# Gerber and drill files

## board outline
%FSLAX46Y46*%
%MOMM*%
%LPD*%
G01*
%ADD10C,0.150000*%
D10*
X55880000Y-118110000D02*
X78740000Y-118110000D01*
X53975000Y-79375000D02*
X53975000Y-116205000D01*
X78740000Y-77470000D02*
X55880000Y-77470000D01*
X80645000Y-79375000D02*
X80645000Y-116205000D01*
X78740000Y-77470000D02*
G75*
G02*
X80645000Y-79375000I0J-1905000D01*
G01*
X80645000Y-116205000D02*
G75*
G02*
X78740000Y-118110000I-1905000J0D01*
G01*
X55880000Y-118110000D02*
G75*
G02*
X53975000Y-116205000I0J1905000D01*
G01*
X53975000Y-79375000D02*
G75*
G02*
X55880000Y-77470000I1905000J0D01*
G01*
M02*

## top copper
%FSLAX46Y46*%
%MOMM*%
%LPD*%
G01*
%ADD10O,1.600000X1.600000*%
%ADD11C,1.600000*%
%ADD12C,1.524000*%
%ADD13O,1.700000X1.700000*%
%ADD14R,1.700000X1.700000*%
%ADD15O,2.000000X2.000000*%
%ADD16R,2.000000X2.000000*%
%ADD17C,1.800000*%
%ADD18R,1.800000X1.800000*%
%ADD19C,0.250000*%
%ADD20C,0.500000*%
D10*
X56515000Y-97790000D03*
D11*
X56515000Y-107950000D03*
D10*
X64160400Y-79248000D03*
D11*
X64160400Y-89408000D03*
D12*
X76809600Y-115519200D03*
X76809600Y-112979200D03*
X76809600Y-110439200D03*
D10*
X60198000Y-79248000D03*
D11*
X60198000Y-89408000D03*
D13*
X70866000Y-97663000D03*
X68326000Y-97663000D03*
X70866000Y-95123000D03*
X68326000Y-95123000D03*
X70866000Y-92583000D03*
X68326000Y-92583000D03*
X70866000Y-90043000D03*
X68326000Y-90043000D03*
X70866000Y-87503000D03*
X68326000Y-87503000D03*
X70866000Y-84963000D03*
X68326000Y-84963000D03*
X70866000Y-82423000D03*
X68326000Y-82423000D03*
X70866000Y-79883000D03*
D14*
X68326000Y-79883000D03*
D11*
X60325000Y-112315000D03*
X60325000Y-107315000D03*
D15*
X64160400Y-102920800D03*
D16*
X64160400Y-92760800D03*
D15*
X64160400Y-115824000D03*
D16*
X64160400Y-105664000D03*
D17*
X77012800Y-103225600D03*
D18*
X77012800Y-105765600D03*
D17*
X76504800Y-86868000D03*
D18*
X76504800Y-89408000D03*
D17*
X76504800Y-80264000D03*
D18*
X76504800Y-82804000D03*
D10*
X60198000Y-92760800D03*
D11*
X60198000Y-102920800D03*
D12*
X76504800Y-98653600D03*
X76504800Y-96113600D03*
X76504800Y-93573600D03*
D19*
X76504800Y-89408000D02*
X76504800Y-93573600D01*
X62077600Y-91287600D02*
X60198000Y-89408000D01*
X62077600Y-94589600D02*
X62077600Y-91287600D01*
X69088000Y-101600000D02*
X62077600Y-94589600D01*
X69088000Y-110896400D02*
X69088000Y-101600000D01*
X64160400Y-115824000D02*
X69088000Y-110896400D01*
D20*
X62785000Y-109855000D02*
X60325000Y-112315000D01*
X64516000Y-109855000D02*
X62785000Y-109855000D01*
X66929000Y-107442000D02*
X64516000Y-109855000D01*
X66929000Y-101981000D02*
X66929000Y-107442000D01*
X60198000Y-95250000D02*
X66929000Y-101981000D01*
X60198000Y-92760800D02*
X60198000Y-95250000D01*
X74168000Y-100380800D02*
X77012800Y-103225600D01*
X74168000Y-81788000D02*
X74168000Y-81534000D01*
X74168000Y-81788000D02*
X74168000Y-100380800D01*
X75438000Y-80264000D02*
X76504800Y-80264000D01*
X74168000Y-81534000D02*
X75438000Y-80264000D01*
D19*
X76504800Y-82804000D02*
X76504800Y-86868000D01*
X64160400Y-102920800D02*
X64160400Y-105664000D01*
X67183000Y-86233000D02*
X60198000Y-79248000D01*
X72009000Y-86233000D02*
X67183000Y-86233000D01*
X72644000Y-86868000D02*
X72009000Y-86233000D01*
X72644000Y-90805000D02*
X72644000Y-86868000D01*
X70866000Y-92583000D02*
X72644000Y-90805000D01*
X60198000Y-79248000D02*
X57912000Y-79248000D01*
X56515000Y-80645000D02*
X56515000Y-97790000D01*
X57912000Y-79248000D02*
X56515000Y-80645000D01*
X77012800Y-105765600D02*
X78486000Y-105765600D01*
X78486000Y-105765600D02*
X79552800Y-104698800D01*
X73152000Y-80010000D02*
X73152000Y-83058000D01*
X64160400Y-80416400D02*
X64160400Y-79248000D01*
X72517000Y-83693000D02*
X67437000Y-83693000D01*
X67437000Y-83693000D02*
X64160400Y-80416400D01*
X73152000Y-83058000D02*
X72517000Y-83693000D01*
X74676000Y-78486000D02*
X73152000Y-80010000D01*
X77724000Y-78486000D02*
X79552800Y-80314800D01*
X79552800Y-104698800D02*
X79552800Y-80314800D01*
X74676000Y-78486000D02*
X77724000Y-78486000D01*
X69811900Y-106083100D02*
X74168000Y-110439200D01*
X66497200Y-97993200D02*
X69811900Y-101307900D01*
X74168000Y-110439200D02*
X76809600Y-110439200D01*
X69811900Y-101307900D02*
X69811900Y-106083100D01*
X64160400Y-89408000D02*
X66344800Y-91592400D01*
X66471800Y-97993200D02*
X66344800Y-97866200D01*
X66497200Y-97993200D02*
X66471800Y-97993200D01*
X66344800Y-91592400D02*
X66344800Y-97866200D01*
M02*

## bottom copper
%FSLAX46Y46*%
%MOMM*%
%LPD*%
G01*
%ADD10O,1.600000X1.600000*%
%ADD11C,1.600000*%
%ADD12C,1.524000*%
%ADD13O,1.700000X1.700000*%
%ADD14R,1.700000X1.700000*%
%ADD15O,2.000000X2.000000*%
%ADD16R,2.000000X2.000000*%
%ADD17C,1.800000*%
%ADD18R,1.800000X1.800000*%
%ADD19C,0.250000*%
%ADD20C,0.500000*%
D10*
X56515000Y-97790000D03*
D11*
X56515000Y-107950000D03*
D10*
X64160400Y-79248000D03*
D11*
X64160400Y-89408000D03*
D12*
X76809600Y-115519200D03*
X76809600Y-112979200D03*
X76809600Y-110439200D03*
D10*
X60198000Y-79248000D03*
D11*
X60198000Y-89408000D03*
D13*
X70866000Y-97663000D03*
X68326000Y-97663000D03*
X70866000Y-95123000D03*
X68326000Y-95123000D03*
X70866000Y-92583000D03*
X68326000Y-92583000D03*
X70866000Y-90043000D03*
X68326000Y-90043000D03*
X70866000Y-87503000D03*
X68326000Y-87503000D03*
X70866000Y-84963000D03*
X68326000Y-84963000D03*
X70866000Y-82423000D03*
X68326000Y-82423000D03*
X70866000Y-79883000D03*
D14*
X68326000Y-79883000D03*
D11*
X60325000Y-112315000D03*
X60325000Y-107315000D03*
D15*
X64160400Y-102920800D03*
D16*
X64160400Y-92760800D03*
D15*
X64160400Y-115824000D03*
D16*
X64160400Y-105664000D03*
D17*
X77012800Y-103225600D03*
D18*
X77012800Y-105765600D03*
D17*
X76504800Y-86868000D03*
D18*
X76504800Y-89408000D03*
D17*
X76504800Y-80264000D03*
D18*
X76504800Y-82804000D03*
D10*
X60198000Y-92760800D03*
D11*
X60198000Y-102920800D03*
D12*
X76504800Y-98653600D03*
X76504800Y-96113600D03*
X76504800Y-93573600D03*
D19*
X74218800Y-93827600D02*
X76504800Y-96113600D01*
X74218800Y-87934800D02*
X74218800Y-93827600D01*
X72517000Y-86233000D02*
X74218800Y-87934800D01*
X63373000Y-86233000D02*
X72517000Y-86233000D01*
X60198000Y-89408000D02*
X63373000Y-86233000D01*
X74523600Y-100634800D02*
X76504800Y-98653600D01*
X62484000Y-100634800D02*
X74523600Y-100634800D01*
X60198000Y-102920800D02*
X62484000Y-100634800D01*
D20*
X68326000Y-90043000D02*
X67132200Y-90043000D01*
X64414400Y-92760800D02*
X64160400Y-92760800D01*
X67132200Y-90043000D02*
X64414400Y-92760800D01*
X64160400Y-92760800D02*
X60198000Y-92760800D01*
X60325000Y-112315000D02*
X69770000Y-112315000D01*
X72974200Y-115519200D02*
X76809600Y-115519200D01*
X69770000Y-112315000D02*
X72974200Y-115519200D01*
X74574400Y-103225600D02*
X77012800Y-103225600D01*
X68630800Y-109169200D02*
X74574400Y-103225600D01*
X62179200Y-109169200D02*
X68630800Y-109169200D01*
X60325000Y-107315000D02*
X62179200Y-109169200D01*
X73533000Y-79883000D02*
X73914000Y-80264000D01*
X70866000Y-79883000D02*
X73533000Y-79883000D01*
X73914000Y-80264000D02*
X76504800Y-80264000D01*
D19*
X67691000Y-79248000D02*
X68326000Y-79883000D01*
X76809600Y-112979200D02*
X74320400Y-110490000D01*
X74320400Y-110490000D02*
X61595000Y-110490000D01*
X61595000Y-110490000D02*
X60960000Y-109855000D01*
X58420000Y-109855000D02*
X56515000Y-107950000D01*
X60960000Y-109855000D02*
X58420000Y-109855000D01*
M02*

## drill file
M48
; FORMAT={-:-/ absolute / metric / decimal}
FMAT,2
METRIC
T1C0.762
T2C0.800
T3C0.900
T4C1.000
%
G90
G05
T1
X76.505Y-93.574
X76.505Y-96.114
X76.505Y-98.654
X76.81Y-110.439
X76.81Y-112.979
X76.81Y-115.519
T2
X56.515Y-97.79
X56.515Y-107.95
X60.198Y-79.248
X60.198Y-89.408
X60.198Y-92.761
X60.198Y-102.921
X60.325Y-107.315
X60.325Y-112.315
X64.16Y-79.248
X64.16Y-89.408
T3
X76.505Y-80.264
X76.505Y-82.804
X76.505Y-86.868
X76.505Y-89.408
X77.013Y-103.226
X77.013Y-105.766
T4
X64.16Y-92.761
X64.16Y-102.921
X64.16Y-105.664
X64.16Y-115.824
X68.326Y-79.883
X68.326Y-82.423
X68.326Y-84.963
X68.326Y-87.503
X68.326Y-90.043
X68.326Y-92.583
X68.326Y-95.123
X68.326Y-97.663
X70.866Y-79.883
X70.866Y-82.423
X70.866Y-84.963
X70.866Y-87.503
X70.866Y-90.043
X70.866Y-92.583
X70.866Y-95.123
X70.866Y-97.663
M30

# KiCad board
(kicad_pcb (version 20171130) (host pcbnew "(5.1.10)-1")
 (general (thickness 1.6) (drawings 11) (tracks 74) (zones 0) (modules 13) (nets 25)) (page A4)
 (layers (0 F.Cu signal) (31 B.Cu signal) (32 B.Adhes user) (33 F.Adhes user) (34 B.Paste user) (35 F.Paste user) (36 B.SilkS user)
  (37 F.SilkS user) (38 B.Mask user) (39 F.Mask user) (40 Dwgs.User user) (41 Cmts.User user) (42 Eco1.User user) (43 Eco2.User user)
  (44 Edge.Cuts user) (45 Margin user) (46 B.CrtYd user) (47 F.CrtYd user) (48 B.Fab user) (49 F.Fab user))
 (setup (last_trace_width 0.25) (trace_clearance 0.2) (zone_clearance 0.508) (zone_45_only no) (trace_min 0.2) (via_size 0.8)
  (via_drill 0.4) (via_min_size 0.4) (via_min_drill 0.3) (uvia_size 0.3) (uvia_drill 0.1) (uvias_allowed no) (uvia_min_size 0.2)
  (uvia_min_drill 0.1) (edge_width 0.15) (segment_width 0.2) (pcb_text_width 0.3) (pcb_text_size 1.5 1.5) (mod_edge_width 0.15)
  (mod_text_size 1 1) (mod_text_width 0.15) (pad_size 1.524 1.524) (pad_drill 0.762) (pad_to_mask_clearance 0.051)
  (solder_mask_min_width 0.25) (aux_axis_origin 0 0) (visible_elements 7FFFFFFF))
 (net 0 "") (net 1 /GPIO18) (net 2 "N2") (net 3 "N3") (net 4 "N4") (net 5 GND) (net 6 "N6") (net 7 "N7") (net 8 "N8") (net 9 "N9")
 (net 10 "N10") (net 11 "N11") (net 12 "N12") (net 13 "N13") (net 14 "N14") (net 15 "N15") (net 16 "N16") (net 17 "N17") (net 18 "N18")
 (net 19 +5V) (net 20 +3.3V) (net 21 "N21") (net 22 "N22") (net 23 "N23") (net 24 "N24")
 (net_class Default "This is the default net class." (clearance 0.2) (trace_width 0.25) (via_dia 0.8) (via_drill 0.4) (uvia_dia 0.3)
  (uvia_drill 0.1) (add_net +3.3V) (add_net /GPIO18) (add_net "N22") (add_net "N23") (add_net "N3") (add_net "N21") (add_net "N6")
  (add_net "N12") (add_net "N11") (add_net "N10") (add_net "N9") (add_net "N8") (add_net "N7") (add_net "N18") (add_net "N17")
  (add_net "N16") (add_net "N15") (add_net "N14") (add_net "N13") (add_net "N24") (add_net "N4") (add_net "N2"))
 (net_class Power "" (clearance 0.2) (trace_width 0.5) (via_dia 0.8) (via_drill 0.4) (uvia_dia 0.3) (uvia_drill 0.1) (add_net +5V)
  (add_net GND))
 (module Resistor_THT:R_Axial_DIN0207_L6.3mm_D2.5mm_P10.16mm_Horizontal (layer F.Cu) (at 56.515 107.95 90)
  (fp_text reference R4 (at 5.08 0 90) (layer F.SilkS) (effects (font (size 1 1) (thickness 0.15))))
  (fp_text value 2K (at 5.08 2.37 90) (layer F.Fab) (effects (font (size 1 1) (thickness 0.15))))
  (pad 2 thru_hole oval (at 10.16 0 90) (size 1.6 1.6) (drill 0.8) (layers *.Cu *.Mask) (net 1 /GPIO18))
  (pad 1 thru_hole circle (at 0 0 90) (size 1.6 1.6) (drill 0.8) (layers *.Cu *.Mask) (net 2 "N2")))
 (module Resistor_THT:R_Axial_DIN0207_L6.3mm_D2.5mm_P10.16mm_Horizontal (layer F.Cu) (at 64.1604 89.408 90)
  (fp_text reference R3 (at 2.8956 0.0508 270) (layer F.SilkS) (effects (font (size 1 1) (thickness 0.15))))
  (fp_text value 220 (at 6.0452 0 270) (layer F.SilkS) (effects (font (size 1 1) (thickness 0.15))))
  (pad 2 thru_hole oval (at 10.16 0 90) (size 1.6 1.6) (drill 0.8) (layers *.Cu *.Mask) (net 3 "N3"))
  (pad 1 thru_hole circle (at 0 0 90) (size 1.6 1.6) (drill 0.8) (layers *.Cu *.Mask) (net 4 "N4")))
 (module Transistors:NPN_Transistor (layer F.Cu) (at 76.8096 110.4392 270)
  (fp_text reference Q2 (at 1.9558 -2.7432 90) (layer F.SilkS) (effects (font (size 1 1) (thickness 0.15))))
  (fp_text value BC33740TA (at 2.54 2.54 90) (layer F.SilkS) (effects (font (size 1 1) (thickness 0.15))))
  (pad 3 thru_hole circle (at 5.08 0 270) (size 1.524 1.524) (drill 0.762) (layers *.Cu *.Mask) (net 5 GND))
  (pad 2 thru_hole circle (at 2.54 0 270) (size 1.524 1.524) (drill 0.762) (layers *.Cu *.Mask) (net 2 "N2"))
  (pad 1 thru_hole circle (at 0 0 270) (size 1.524 1.524) (drill 0.762) (layers *.Cu *.Mask) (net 4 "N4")))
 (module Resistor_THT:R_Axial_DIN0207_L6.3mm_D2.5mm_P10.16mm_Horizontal (layer F.Cu) (at 60.198 89.408 90)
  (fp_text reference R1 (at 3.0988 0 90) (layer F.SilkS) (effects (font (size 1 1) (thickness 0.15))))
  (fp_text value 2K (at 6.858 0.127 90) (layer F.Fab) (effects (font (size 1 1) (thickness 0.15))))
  (pad 2 thru_hole oval (at 10.16 0 90) (size 1.6 1.6) (drill 0.8) (layers *.Cu *.Mask) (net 1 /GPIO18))
  (pad 1 thru_hole circle (at 0 0 90) (size 1.6 1.6) (drill 0.8) (layers *.Cu *.Mask) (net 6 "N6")))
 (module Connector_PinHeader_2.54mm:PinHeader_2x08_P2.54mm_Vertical (layer F.Cu) (at 68.326 79.883)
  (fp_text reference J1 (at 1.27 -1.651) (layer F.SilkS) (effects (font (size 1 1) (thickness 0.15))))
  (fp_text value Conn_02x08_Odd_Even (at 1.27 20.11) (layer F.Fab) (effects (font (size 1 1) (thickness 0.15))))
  (pad 16 thru_hole oval (at 2.54 17.78) (size 1.7 1.7) (drill 1) (layers *.Cu *.Mask) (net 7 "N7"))
  (pad 15 thru_hole oval (at 0 17.78) (size 1.7 1.7) (drill 1) (layers *.Cu *.Mask) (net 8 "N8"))
  (pad 14 thru_hole oval (at 2.54 15.24) (size 1.7 1.7) (drill 1) (layers *.Cu *.Mask) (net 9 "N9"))
  (pad 13 thru_hole oval (at 0 15.24) (size 1.7 1.7) (drill 1) (layers *.Cu *.Mask) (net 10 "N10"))
  (pad 12 thru_hole oval (at 2.54 12.7) (size 1.7 1.7) (drill 1) (layers *.Cu *.Mask) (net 1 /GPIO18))
  (pad 11 thru_hole oval (at 0 12.7) (size 1.7 1.7) (drill 1) (layers *.Cu *.Mask) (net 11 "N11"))
  (pad 10 thru_hole oval (at 2.54 10.16) (size 1.7 1.7) (drill 1) (layers *.Cu *.Mask) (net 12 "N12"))
  (pad 9 thru_hole oval (at 0 10.16) (size 1.7 1.7) (drill 1) (layers *.Cu *.Mask) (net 5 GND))
  (pad 8 thru_hole oval (at 2.54 7.62) (size 1.7 1.7) (drill 1) (layers *.Cu *.Mask) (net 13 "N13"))
  (pad 7 thru_hole oval (at 0 7.62) (size 1.7 1.7) (drill 1) (layers *.Cu *.Mask) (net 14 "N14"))
  (pad 6 thru_hole oval (at 2.54 5.08) (size 1.7 1.7) (drill 1) (layers *.Cu *.Mask) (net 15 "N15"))
  (pad 5 thru_hole oval (at 0 5.08) (size 1.7 1.7) (drill 1) (layers *.Cu *.Mask) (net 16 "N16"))
  (pad 4 thru_hole oval (at 2.54 2.54) (size 1.7 1.7) (drill 1) (layers *.Cu *.Mask) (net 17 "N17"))
  (pad 3 thru_hole oval (at 0 2.54) (size 1.7 1.7) (drill 1) (layers *.Cu *.Mask) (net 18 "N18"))
  (pad 2 thru_hole oval (at 2.54 0) (size 1.7 1.7) (drill 1) (layers *.Cu *.Mask) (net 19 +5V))
  (pad 1 thru_hole rect (at 0 0) (size 1.7 1.7) (drill 1) (layers *.Cu *.Mask) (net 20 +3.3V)))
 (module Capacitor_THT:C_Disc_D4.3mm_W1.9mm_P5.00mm (layer F.Cu) (at 60.325 107.315 270)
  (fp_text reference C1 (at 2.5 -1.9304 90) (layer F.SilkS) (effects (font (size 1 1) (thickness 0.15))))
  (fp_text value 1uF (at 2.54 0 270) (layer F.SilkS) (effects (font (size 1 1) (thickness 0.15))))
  (pad 2 thru_hole circle (at 5 0 270) (size 1.6 1.6) (drill 0.8) (layers *.Cu *.Mask) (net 5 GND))
  (pad 1 thru_hole circle (at 0 0 270) (size 1.6 1.6) (drill 0.8) (layers *.Cu *.Mask) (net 19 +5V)))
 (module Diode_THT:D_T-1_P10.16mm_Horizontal (layer F.Cu) (at 64.1604 92.7608 270)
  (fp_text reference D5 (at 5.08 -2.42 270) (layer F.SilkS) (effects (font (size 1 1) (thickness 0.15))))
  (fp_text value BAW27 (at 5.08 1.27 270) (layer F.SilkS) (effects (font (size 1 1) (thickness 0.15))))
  (pad 2 thru_hole oval (at 10.16 0 270) (size 2 2) (drill 1) (layers *.Cu *.Mask) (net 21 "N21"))
  (pad 1 thru_hole rect (at 0 0 270) (size 2 2) (drill 1) (layers *.Cu *.Mask) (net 5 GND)))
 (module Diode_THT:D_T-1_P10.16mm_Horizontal (layer F.Cu) (at 64.1604 105.664 270)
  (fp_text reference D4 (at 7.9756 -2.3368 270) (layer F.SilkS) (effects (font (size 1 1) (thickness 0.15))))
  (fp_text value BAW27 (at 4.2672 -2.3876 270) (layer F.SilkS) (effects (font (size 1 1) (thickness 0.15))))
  (pad 2 thru_hole oval (at 10.16 0 270) (size 2 2) (drill 1) (layers *.Cu *.Mask) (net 6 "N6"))
  (pad 1 thru_hole rect (at 0 0 270) (size 2 2) (drill 1) (layers *.Cu *.Mask) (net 21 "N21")))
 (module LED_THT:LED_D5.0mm (layer F.Cu) (at 77.0128 105.7656 90)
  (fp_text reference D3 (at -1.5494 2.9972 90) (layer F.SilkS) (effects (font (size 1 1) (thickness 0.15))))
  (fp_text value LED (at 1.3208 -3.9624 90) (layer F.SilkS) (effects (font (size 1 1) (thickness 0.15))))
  (pad 2 thru_hole circle (at 2.54 0 90) (size 1.8 1.8) (drill 0.9) (layers *.Cu *.Mask) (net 19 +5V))
  (pad 1 thru_hole rect (at 0 0 90) (size 1.8 1.8) (drill 0.9) (layers *.Cu *.Mask) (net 3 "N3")))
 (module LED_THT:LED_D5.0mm (layer F.Cu) (at 76.5048 89.408 90)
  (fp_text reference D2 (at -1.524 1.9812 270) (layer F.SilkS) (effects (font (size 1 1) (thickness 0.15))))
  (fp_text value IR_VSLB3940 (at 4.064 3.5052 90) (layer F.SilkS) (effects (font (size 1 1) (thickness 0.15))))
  (pad 2 thru_hole circle (at 2.54 0 90) (size 1.8 1.8) (drill 0.9) (layers *.Cu *.Mask) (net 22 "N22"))
  (pad 1 thru_hole rect (at 0 0 90) (size 1.8 1.8) (drill 0.9) (layers *.Cu *.Mask) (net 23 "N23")))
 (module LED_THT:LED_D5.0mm (layer F.Cu) (at 76.5048 82.804 90)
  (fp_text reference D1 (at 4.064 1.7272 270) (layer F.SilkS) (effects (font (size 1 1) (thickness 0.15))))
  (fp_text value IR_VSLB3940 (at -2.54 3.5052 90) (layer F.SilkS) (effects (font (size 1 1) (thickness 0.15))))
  (pad 2 thru_hole circle (at 2.54 0 90) (size 1.8 1.8) (drill 0.9) (layers *.Cu *.Mask) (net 19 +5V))
  (pad 1 thru_hole rect (at 0 0 90) (size 1.8 1.8) (drill 0.9) (layers *.Cu *.Mask) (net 22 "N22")))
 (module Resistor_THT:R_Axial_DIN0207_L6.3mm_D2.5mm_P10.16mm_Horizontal (layer F.Cu) (at 60.198 102.9208 90)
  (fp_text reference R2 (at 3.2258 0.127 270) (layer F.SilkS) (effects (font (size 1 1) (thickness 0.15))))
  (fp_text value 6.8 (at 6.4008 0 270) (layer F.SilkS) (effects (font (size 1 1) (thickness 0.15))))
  (pad 2 thru_hole oval (at 10.16 0 90) (size 1.6 1.6) (drill 0.8) (layers *.Cu *.Mask) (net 5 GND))
  (pad 1 thru_hole circle (at 0 0 90) (size 1.6 1.6) (drill 0.8) (layers *.Cu *.Mask) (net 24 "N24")))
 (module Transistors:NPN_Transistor (layer F.Cu) (at 76.5048 93.5736 270)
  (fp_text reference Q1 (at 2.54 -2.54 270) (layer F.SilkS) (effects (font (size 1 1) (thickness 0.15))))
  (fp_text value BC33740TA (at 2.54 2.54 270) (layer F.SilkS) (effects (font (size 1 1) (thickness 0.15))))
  (pad 3 thru_hole circle (at 5.08 0 270) (size 1.524 1.524) (drill 0.762) (layers *.Cu *.Mask) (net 24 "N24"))
  (pad 2 thru_hole circle (at 2.54 0 270) (size 1.524 1.524) (drill 0.762) (layers *.Cu *.Mask) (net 6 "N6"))
  (pad 1 thru_hole circle (at 0 0 270) (size 1.524 1.524) (drill 0.762) (layers *.Cu *.Mask) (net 23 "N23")))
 (gr_line (start 55.88 118.11) (end 78.74 118.11) (layer Edge.Cuts) (width 0.15))
 (gr_line (start 53.975 79.375) (end 53.975 116.205) (layer Edge.Cuts) (width 0.15))
 (gr_line (start 78.74 77.47) (end 55.88 77.47) (layer Edge.Cuts) (width 0.15))
 (gr_line (start 80.645 79.375) (end 80.645 116.205) (layer Edge.Cuts) (width 0.15))
 (gr_arc (start 78.74 79.375) (end 80.645 79.375) (angle -90) (layer Edge.Cuts) (width 0.15))
 (gr_arc (start 78.74 116.205) (end 78.74 118.11) (angle -90) (layer Edge.Cuts) (width 0.15))
 (gr_arc (start 55.88 116.205) (end 53.975 116.205) (angle -90) (layer Edge.Cuts) (width 0.15))
 (gr_arc (start 55.88 79.375) (end 55.88 77.47) (angle -90) (layer Edge.Cuts) (width 0.15))
 (segment (start 76.5048 89.408) (end 76.5048 93.5736) (width 0.25) (layer F.Cu) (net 23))
 (segment (start 74.2188 93.8276) (end 76.5048 96.1136) (width 0.25) (layer B.Cu) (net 6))
 (segment (start 74.2188 87.9348) (end 74.2188 93.8276) (width 0.25) (layer B.Cu) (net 6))
 (segment (start 72.517 86.233) (end 74.2188 87.9348) (width 0.25) (layer B.Cu) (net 6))
 (segment (start 63.373 86.233) (end 72.517 86.233) (width 0.25) (layer B.Cu) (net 6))
 (segment (start 60.198 89.408) (end 63.373 86.233) (width 0.25) (layer B.Cu) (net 6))
 (segment (start 62.0776 91.2876) (end 60.198 89.408) (width 0.25) (layer F.Cu) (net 6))
 (segment (start 62.0776 94.5896) (end 62.0776 91.2876) (width 0.25) (layer F.Cu) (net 6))
 (segment (start 69.088 101.6) (end 62.0776 94.5896) (width 0.25) (layer F.Cu) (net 6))
 (segment (start 69.088 110.8964) (end 69.088 101.6) (width 0.25) (layer F.Cu) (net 6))
 (segment (start 64.1604 115.824) (end 69.088 110.8964) (width 0.25) (layer F.Cu) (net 6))
 (segment (start 74.5236 100.6348) (end 76.5048 98.6536) (width 0.25) (layer B.Cu) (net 24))
 (segment (start 62.484 100.6348) (end 74.5236 100.6348) (width 0.25) (layer B.Cu) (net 24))
 (segment (start 60.198 102.9208) (end 62.484 100.6348) (width 0.25) (layer B.Cu) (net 24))
 (segment (start 68.326 90.043) (end 67.1322 90.043) (width 0.5) (layer B.Cu) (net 5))
 (segment (start 64.4144 92.7608) (end 64.1604 92.7608) (width 0.5) (layer B.Cu) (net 5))
 (segment (start 67.1322 90.043) (end 64.4144 92.7608) (width 0.5) (layer B.Cu) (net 5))
 (segment (start 64.1604 92.7608) (end 60.198 92.7608) (width 0.5) (layer B.Cu) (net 5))
 (segment (start 60.325 112.315) (end 69.77 112.315) (width 0.5) (layer B.Cu) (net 5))
 (segment (start 72.9742 115.5192) (end 76.8096 115.5192) (width 0.5) (layer B.Cu) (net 5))
 (segment (start 69.77 112.315) (end 72.9742 115.5192) (width 0.5) (layer B.Cu) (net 5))
 (segment (start 62.785 109.855) (end 60.325 112.315) (width 0.5) (layer F.Cu) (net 5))
 (segment (start 64.516 109.855) (end 62.785 109.855) (width 0.5) (layer F.Cu) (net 5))
 (segment (start 66.929 107.442) (end 64.516 109.855) (width 0.5) (layer F.Cu) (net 5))
 (segment (start 66.929 101.981) (end 66.929 107.442) (width 0.5) (layer F.Cu) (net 5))
 (segment (start 60.198 95.25) (end 66.929 101.981) (width 0.5) (layer F.Cu) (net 5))
 (segment (start 60.198 92.7608) (end 60.198 95.25) (width 0.5) (layer F.Cu) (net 5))
 (segment (start 74.168 100.3808) (end 77.0128 103.2256) (width 0.5) (layer F.Cu) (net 19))
 (segment (start 74.5744 103.2256) (end 77.0128 103.2256) (width 0.5) (layer B.Cu) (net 19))
 (segment (start 68.6308 109.1692) (end 74.5744 103.2256) (width 0.5) (layer B.Cu) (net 19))
 (segment (start 62.1792 109.1692) (end 68.6308 109.1692) (width 0.5) (layer B.Cu) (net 19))
 (segment (start 60.325 107.315) (end 62.1792 109.1692) (width 0.5) (layer B.Cu) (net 19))
 (segment (start 74.168 81.788) (end 74.168 81.534) (width 0.5) (layer F.Cu) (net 19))
 (segment (start 74.168 81.788) (end 74.168 100.3808) (width 0.5) (layer F.Cu) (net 19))
 (segment (start 75.438 80.264) (end 76.5048 80.264) (width 0.5) (layer F.Cu) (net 19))
 (segment (start 74.168 81.534) (end 75.438 80.264) (width 0.5) (layer F.Cu) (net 19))
 (segment (start 73.533 79.883) (end 73.914 80.264) (width 0.5) (layer B.Cu) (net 19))
 (segment (start 70.866 79.883) (end 73.533 79.883) (width 0.5) (layer B.Cu) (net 19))
 (segment (start 73.914 80.264) (end 76.5048 80.264) (width 0.5) (layer B.Cu) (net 19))
 (segment (start 76.5048 82.804) (end 76.5048 86.868) (width 0.25) (layer F.Cu) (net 22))
 (segment (start 64.1604 102.9208) (end 64.1604 105.664) (width 0.25) (layer F.Cu) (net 21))
 (segment (start 67.183 86.233) (end 60.198 79.248) (width 0.25) (layer F.Cu) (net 1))
 (segment (start 72.009 86.233) (end 67.183 86.233) (width 0.25) (layer F.Cu) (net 1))
 (segment (start 72.644 86.868) (end 72.009 86.233) (width 0.25) (layer F.Cu) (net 1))
 (segment (start 72.644 90.805) (end 72.644 86.868) (width 0.25) (layer F.Cu) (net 1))
 (segment (start 70.866 92.583) (end 72.644 90.805) (width 0.25) (layer F.Cu) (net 1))
 (segment (start 60.198 79.248) (end 57.912 79.248) (width 0.25) (layer F.Cu) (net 1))
 (segment (start 56.515 80.645) (end 56.515 97.79) (width 0.25) (layer F.Cu) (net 1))
 (segment (start 57.912 79.248) (end 56.515 80.645) (width 0.25) (layer F.Cu) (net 1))
 (segment (start 67.691 79.248) (end 68.326 79.883) (width 0.25) (layer B.Cu) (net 20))
 (segment (start 77.0128 105.7656) (end 78.486 105.7656) (width 0.25) (layer F.Cu) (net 3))
 (segment (start 78.486 105.7656) (end 79.5528 104.6988) (width 0.25) (layer F.Cu) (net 3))
 (segment (start 73.152 80.01) (end 73.152 83.058) (width 0.25) (layer F.Cu) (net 3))
 (segment (start 64.1604 80.4164) (end 64.1604 79.248) (width 0.25) (layer F.Cu) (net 3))
 (segment (start 72.517 83.693) (end 67.437 83.693) (width 0.25) (layer F.Cu) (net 3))
 (segment (start 67.437 83.693) (end 64.1604 80.4164) (width 0.25) (layer F.Cu) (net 3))
 (segment (start 73.152 83.058) (end 72.517 83.693) (width 0.25) (layer F.Cu) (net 3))
 (segment (start 74.676 78.486) (end 73.152 80.01) (width 0.25) (layer F.Cu) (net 3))
 (segment (start 77.724 78.486) (end 79.5528 80.3148) (width 0.25) (layer F.Cu) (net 3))
 (segment (start 79.5528 104.6988) (end 79.5528 80.3148) (width 0.25) (layer F.Cu) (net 3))
 (segment (start 74.676 78.486) (end 77.724 78.486) (width 0.25) (layer F.Cu) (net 3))
 (segment (start 69.8119 106.0831) (end 74.168 110.4392) (width 0.25) (layer F.Cu) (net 4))
 (segment (start 66.4972 97.9932) (end 69.8119 101.3079) (width 0.25) (layer F.Cu) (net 4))
 (segment (start 74.168 110.4392) (end 76.8096 110.4392) (width 0.25) (layer F.Cu) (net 4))
 (segment (start 69.8119 101.3079) (end 69.8119 106.0831) (width 0.25) (layer F.Cu) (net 4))
 (segment (start 64.1604 89.408) (end 66.3448 91.5924) (width 0.25) (layer F.Cu) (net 4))
 (segment (start 66.4718 97.9932) (end 66.3448 97.8662) (width 0.25) (layer F.Cu) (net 4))
 (segment (start 66.4972 97.9932) (end 66.4718 97.9932) (width 0.25) (layer F.Cu) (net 4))
 (segment (start 66.3448 91.5924) (end 66.3448 97.8662) (width 0.25) (layer F.Cu) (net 4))
 (segment (start 76.8096 112.9792) (end 74.3204 110.49) (width 0.25) (layer B.Cu) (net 2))
 (segment (start 74.3204 110.49) (end 61.595 110.49) (width 0.25) (layer B.Cu) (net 2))
 (segment (start 61.595 110.49) (end 60.96 109.855) (width 0.25) (layer B.Cu) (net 2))
 (segment (start 58.42 109.855) (end 56.515 107.95) (width 0.25) (layer B.Cu) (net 2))
 (segment (start 60.96 109.855) (end 58.42 109.855) (width 0.25) (layer B.Cu) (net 2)))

